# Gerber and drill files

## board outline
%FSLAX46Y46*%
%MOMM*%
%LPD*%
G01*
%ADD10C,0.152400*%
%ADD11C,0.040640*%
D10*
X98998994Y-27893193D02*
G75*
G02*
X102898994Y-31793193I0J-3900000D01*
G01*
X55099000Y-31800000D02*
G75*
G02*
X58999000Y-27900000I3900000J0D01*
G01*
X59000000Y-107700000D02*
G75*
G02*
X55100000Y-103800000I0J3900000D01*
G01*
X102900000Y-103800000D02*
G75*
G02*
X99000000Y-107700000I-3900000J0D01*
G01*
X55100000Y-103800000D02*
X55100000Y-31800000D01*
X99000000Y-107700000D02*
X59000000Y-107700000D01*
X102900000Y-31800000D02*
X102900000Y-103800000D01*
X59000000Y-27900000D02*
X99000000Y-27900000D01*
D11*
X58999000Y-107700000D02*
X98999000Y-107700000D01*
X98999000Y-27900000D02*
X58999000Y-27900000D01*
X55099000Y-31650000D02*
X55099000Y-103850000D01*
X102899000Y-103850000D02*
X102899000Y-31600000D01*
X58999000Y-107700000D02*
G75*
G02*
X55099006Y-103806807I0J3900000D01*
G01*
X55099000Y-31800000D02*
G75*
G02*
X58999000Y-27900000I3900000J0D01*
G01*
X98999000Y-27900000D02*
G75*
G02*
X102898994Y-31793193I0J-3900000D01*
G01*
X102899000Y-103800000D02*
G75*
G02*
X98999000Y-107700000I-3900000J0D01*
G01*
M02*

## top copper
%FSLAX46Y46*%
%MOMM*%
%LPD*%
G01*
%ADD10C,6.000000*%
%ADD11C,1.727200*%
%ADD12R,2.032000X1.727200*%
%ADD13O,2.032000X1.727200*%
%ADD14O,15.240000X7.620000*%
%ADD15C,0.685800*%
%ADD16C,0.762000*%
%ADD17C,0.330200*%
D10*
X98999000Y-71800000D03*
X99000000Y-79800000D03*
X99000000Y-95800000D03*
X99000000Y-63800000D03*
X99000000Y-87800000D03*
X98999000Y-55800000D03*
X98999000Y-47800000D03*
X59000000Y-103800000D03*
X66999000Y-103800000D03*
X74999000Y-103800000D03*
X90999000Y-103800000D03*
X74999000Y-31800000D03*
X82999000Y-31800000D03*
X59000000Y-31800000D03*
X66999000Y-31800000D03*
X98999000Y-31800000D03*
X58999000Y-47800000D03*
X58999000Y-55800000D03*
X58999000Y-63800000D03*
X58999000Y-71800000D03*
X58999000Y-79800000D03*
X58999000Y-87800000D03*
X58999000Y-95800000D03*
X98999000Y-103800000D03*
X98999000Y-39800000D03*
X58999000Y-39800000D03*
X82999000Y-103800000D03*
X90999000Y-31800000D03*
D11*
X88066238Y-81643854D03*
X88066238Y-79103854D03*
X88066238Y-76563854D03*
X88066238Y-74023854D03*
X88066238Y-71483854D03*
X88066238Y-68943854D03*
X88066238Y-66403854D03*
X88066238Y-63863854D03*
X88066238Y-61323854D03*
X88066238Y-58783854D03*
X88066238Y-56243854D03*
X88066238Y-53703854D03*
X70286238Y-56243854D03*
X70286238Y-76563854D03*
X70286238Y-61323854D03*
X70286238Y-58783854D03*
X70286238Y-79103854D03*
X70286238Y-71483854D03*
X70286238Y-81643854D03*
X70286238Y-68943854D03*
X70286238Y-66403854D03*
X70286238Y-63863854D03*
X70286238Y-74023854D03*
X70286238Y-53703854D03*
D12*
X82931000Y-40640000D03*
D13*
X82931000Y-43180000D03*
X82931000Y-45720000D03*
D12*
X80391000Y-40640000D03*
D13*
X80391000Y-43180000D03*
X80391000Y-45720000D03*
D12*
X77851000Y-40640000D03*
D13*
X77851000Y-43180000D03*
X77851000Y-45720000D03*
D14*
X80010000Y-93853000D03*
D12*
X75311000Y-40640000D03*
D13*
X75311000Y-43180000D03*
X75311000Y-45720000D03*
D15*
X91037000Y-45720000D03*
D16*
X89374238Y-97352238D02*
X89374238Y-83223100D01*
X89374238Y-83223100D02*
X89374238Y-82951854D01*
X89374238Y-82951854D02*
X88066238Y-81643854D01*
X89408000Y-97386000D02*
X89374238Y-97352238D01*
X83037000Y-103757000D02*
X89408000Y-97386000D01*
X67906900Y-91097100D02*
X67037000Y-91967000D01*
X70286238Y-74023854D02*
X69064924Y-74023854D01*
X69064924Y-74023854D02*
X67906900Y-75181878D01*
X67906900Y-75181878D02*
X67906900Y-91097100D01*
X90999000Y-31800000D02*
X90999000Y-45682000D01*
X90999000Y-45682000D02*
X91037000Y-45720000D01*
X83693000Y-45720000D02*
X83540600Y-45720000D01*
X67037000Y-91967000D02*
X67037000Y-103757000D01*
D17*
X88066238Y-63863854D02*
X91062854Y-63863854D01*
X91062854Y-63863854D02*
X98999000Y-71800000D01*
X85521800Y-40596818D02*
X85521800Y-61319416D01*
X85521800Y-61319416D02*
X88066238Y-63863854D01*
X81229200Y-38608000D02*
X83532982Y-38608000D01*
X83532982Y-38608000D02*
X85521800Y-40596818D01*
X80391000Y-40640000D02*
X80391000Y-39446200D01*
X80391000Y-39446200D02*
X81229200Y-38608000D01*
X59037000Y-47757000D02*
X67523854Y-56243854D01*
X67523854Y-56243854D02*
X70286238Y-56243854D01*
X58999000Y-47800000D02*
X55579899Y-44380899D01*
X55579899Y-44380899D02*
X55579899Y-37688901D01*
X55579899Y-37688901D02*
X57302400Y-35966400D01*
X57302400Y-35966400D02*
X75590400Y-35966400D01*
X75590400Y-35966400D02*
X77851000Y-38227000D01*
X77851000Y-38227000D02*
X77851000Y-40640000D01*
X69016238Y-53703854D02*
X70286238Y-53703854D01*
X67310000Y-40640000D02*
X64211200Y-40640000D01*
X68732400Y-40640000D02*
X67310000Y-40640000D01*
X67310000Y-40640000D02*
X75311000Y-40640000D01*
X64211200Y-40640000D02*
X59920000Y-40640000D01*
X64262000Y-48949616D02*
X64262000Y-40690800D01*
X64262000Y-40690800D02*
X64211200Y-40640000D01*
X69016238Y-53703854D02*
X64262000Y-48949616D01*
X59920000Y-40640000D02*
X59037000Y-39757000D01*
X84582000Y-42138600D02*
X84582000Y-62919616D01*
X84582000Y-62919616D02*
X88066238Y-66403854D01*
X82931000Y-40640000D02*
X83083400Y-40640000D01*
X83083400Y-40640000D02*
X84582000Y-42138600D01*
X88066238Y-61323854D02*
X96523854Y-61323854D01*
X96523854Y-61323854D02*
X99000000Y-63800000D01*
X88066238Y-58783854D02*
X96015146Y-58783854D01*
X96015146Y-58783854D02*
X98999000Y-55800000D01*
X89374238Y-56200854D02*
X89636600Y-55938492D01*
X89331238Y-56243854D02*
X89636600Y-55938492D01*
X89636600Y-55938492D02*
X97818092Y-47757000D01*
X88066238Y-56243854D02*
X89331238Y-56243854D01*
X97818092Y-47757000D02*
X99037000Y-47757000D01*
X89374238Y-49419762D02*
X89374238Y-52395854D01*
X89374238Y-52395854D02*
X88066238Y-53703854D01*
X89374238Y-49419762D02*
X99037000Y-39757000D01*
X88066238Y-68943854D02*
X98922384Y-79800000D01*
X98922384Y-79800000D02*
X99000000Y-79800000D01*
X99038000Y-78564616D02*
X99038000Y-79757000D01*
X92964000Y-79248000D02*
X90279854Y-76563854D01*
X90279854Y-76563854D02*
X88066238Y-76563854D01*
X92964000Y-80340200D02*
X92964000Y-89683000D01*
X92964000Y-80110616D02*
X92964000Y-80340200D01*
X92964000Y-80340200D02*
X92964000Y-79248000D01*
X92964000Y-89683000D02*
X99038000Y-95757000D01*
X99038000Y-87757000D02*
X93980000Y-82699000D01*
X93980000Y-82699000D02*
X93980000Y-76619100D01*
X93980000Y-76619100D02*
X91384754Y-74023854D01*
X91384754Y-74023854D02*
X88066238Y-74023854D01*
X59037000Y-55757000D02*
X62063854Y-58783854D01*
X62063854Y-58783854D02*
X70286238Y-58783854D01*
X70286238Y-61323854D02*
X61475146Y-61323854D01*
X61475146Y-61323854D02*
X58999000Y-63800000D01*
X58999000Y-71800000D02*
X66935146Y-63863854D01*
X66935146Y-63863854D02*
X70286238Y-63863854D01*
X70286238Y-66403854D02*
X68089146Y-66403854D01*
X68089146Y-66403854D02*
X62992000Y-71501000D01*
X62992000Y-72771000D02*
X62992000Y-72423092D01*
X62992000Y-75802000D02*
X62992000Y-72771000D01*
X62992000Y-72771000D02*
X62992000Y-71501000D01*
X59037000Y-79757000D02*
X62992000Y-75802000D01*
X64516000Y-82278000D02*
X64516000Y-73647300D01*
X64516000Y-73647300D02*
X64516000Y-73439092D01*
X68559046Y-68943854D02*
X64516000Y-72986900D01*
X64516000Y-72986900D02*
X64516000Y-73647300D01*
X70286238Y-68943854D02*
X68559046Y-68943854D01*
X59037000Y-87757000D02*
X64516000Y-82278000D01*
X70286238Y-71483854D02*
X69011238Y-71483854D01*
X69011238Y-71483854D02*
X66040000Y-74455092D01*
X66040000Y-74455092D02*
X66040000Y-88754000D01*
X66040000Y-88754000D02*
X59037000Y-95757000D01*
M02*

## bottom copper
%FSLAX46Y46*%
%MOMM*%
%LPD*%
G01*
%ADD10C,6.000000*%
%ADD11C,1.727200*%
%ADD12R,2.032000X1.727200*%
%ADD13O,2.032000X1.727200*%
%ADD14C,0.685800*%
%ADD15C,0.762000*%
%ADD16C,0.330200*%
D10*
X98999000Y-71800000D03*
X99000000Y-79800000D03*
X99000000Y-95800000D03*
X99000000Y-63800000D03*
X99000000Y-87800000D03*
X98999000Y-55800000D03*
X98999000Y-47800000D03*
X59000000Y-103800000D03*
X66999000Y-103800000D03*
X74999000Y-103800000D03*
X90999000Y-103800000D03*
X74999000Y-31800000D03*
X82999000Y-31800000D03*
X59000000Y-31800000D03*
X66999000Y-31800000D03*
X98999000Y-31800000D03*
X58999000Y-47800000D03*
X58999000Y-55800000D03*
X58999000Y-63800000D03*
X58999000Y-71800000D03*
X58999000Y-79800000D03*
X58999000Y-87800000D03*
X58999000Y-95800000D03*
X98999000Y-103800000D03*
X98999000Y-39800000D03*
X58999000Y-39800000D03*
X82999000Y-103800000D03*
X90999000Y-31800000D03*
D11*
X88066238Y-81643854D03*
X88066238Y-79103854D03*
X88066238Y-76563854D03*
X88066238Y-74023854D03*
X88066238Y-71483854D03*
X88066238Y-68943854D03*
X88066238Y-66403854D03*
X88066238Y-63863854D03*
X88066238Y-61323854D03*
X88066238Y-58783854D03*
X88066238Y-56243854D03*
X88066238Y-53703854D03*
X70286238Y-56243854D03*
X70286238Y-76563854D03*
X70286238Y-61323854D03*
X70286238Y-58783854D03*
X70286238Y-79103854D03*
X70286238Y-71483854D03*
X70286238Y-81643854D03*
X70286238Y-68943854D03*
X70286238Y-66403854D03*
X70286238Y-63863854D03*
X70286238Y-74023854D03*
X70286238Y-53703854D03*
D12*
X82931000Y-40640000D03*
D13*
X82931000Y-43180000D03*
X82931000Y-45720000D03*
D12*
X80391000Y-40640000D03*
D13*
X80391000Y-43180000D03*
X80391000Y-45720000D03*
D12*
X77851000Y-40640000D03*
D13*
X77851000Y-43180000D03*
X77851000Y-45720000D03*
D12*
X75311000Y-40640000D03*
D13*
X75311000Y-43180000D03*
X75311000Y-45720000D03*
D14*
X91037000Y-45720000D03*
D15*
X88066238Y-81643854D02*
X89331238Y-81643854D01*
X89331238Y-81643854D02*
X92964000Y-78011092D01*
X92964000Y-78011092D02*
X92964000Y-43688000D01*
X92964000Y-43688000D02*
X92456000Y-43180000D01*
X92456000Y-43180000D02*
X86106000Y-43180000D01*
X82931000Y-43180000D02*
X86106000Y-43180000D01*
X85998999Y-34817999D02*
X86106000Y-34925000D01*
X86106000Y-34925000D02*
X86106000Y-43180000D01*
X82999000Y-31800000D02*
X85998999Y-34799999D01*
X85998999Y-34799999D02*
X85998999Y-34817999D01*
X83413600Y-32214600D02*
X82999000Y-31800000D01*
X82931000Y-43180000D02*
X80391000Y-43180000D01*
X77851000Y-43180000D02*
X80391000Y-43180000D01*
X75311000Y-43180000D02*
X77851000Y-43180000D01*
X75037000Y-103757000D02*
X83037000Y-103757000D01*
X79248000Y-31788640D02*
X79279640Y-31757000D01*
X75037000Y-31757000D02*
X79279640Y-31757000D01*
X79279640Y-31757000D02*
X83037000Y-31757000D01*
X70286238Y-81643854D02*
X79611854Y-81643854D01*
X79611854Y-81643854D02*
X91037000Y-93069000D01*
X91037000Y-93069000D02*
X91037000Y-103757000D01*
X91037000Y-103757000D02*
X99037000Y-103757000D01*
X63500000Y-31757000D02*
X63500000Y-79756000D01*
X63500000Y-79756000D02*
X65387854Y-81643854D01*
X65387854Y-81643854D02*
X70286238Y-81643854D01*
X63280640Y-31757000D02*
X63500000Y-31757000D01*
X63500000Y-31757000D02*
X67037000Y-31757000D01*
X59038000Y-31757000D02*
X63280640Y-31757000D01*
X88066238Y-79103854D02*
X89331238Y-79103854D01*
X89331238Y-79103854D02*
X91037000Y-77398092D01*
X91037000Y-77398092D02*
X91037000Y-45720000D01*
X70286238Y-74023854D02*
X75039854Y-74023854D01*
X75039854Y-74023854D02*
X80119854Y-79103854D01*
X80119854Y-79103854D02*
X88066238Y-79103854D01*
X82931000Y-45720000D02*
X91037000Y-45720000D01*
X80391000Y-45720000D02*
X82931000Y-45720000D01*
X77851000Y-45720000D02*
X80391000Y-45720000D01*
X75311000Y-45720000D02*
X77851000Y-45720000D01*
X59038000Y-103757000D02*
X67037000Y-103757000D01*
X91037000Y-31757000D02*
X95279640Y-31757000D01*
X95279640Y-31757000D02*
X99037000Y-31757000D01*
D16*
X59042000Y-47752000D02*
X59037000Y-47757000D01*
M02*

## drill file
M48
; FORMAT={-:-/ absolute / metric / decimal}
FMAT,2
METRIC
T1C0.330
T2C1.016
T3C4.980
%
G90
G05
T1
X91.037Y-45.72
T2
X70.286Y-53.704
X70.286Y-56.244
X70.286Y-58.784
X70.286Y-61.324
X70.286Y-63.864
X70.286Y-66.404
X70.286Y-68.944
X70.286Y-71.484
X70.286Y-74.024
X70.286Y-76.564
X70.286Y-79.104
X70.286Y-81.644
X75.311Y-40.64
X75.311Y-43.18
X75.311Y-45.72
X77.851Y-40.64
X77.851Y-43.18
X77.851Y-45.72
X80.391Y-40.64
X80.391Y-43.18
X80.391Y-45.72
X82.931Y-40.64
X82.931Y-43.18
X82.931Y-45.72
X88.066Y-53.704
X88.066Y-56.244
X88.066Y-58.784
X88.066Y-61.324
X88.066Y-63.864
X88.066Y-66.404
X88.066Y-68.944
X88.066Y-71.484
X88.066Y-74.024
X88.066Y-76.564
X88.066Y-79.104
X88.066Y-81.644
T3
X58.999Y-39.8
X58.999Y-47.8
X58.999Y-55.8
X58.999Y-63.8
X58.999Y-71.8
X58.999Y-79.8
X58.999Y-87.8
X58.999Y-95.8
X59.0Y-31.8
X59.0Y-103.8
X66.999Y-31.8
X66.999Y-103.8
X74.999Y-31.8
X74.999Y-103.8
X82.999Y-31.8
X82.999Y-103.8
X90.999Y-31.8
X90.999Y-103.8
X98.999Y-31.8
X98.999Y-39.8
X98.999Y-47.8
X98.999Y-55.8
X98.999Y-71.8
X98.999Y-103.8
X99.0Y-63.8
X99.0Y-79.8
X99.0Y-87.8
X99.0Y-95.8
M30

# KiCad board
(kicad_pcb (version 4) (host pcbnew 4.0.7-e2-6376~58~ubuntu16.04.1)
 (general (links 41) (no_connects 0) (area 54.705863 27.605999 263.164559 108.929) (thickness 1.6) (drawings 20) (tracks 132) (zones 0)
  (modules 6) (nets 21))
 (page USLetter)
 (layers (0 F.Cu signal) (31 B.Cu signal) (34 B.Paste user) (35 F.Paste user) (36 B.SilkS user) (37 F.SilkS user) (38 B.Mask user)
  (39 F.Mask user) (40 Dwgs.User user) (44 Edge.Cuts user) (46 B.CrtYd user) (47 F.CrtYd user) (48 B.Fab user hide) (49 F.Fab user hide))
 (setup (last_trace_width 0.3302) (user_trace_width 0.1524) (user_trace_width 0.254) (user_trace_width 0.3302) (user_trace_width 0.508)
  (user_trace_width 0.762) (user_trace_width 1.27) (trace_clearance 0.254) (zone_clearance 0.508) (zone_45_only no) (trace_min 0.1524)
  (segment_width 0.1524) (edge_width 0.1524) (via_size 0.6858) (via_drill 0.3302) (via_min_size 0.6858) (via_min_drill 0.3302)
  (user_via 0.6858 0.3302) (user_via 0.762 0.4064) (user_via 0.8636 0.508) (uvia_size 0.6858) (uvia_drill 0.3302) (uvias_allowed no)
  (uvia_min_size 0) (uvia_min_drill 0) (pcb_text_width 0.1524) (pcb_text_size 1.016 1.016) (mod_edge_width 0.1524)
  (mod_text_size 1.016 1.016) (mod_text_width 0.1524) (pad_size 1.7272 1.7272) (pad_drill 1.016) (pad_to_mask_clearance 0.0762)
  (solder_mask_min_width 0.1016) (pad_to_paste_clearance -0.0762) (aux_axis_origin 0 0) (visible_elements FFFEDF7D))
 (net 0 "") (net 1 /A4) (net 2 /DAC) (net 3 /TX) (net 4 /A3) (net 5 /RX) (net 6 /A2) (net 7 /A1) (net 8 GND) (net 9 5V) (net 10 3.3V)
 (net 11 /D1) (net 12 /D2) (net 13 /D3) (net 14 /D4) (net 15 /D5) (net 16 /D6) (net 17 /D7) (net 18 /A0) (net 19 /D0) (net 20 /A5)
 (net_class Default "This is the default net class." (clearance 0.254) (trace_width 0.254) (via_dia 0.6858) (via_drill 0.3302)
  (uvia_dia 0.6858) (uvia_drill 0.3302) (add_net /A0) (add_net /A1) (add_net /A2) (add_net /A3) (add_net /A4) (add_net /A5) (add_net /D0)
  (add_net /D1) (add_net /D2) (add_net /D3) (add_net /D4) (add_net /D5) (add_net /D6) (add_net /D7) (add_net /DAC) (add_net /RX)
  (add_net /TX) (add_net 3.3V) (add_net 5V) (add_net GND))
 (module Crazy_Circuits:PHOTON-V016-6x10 (layer F.Cu) (at 58.999 103.8)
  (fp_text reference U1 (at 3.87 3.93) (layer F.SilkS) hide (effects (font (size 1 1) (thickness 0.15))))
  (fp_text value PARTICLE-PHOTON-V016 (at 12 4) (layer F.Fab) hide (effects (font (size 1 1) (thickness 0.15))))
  (fp_line (start 0 3.9) (end 40 3.9) (layer Edge.Cuts) (width 0.04064))
  (fp_line (start 40 -75.9) (end 0 -75.9) (layer Edge.Cuts) (width 0.04064))
  (fp_line (start -3.9 -72.15) (end -3.9 0.05) (layer Edge.Cuts) (width 0.04064))
  (fp_line (start 43.9 0.05) (end 43.9 -72.2) (layer Edge.Cuts) (width 0.04064))
  (fp_arc (start 0 0) (end 0 3.9) (angle 89.9) (layer Edge.Cuts) (width 0.04064))
  (fp_arc (start 0 -72) (end -3.9 -72) (angle 90) (layer Edge.Cuts) (width 0.04064))
  (fp_arc (start 40 -72) (end 40 -75.9) (angle 89.9) (layer Edge.Cuts) (width 0.04064))
  (fp_arc (start 40 0) (end 43.9 0) (angle 90) (layer Edge.Cuts) (width 0.04064))
  (pad A4 thru_hole circle (at 40 -32 90) (size 6 6) (drill 4.98) (layers *.Cu *.Mask) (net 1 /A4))
  (pad DAC thru_hole circle (at 40.001 -24 90) (size 6 6) (drill 4.98) (layers *.Cu *.Mask) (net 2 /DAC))
  (pad TX thru_hole circle (at 40.001 -8 90) (size 6 6) (drill 4.98) (layers *.Cu *.Mask) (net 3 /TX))
  (pad A3 thru_hole circle (at 40.001 -40 90) (size 6 6) (drill 4.98) (layers *.Cu *.Mask) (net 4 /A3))
  (pad RX thru_hole circle (at 40.001 -16 90) (size 6 6) (drill 4.98) (layers *.Cu *.Mask) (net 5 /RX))
  (pad A2 thru_hole circle (at 40 -48 90) (size 6 6) (drill 4.98) (layers *.Cu *.Mask) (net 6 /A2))
  (pad A1 thru_hole circle (at 40 -56 90) (size 6 6) (drill 4.98) (layers *.Cu *.Mask) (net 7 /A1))
  (pad GND thru_hole circle (at 0.001 0 90) (size 6 6) (drill 4.98) (layers *.Cu *.Mask) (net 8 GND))
  (pad GND thru_hole circle (at 8 0 90) (size 6 6) (drill 4.98) (layers *.Cu *.Mask) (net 8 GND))
  (pad 5V thru_hole circle (at 16 0 90) (size 6 6) (drill 4.98) (layers *.Cu *.Mask) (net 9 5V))
  (pad 3V thru_hole circle (at 32 0 90) (size 6 6) (drill 4.98) (layers *.Cu *.Mask) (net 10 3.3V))
  (pad 5V thru_hole circle (at 16 -72 90) (size 6 6) (drill 4.98) (layers *.Cu *.Mask) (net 9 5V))
  (pad 5V thru_hole circle (at 24 -72 90) (size 6 6) (drill 4.98) (layers *.Cu *.Mask) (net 9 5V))
  (pad 3V thru_hole circle (at 0.001 -72 90) (size 6 6) (drill 4.98) (layers *.Cu *.Mask) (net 10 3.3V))
  (pad 3V thru_hole circle (at 8 -72 90) (size 6 6) (drill 4.98) (layers *.Cu *.Mask) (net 10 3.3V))
  (pad GND thru_hole circle (at 40 -72 90) (size 6 6) (drill 4.98) (layers *.Cu *.Mask) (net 8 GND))
  (pad D1 thru_hole circle (at 0 -56 90) (size 6 6) (drill 4.98) (layers *.Cu *.Mask) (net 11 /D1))
  (pad D2 thru_hole circle (at 0 -48 90) (size 6 6) (drill 4.98) (layers *.Cu *.Mask) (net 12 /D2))
  (pad D3 thru_hole circle (at 0 -40 90) (size 6 6) (drill 4.98) (layers *.Cu *.Mask) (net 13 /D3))
  (pad D4 thru_hole circle (at 0 -32 90) (size 6 6) (drill 4.98) (layers *.Cu *.Mask) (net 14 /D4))
  (pad D5 thru_hole circle (at 0 -24 90) (size 6 6) (drill 4.98) (layers *.Cu *.Mask) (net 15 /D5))
  (pad D6 thru_hole circle (at 0 -16 90) (size 6 6) (drill 4.98) (layers *.Cu *.Mask) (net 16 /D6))
  (pad D7 thru_hole circle (at 0 -8 90) (size 6 6) (drill 4.98) (layers *.Cu *.Mask) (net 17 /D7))
  (pad 3V thru_hole circle (at 40 0 90) (size 6 6) (drill 4.98) (layers *.Cu *.Mask) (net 10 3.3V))
  (pad A0 thru_hole circle (at 40 -64 90) (size 6 6) (drill 4.98) (layers *.Cu *.Mask) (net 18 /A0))
  (pad D0 thru_hole circle (at 0 -64 90) (size 6 6) (drill 4.98) (layers *.Cu *.Mask) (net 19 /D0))
  (pad 5V thru_hole circle (at 24 0 90) (size 6 6) (drill 4.98) (layers *.Cu *.Mask) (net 9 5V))
  (pad GND thru_hole circle (at 32 -72 90) (size 6 6) (drill 4.98) (layers *.Cu *.Mask) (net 8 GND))
  (pad VIN thru_hole circle (at 29.067238 -22.156146 180) (size 1.7272 1.7272) (drill 1.016) (layers *.Cu *.Mask F.SilkS) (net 9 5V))
  (pad GND thru_hole circle (at 29.067238 -24.696146 180) (size 1.7272 1.7272) (drill 1.016) (layers *.Cu *.Mask F.SilkS) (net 8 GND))
  (pad TX thru_hole circle (at 29.067238 -27.236146 180) (size 1.7272 1.7272) (drill 1.016) (layers *.Cu *.Mask F.SilkS) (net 3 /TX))
  (pad RX thru_hole circle (at 29.067238 -29.776146 180) (size 1.7272 1.7272) (drill 1.016) (layers *.Cu *.Mask F.SilkS) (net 5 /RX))
  (pad WKP thru_hole circle (at 29.067238 -32.316146 180) (size 1.7272 1.7272) (drill 1.016) (layers *.Cu *.Mask F.SilkS))
  (pad DAC thru_hole circle (at 29.067238 -34.856146 180) (size 1.7272 1.7272) (drill 1.016) (layers *.Cu *.Mask F.SilkS) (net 2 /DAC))
  (pad A5 thru_hole circle (at 29.067238 -37.396146 180) (size 1.7272 1.7272) (drill 1.016) (layers *.Cu *.Mask F.SilkS) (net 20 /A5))
  (pad A4 thru_hole circle (at 29.067238 -39.936146 180) (size 1.7272 1.7272) (drill 1.016) (layers *.Cu *.Mask F.SilkS) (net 1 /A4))
  (pad A3 thru_hole circle (at 29.067238 -42.476146 180) (size 1.7272 1.7272) (drill 1.016) (layers *.Cu *.Mask F.SilkS) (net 4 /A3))
  (pad A2 thru_hole circle (at 29.067238 -45.016146 180) (size 1.7272 1.7272) (drill 1.016) (layers *.Cu *.Mask F.SilkS) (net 6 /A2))
  (pad A1 thru_hole circle (at 29.067238 -47.556146 180) (size 1.7272 1.7272) (drill 1.016) (layers *.Cu *.Mask F.SilkS) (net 7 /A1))
  (pad A0 thru_hole circle (at 29.067238 -50.096146 180) (size 1.7272 1.7272) (drill 1.016) (layers *.Cu *.Mask F.SilkS) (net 18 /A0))
  (pad D1 thru_hole circle (at 11.287238 -47.556146 180) (size 1.7272 1.7272) (drill 1.016) (layers *.Cu *.Mask F.SilkS) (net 11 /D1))
  (pad VBAT thru_hole circle (at 11.287238 -27.236146 180) (size 1.7272 1.7272) (drill 1.016) (layers *.Cu *.Mask F.SilkS))
  (pad D3 thru_hole circle (at 11.287238 -42.476146 180) (size 1.7272 1.7272) (drill 1.016) (layers *.Cu *.Mask F.SilkS) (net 13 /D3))
  (pad D2 thru_hole circle (at 11.287238 -45.016146 180) (size 1.7272 1.7272) (drill 1.016) (layers *.Cu *.Mask F.SilkS) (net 12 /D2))
  (pad RST thru_hole circle (at 11.287238 -24.696146 180) (size 1.7272 1.7272) (drill 1.016) (layers *.Cu *.Mask F.SilkS))
  (pad D7 thru_hole circle (at 11.287238 -32.316146 180) (size 1.7272 1.7272) (drill 1.016) (layers *.Cu *.Mask F.SilkS) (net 17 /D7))
  (pad 3V thru_hole circle (at 11.287238 -22.156146 180) (size 1.7272 1.7272) (drill 1.016) (layers *.Cu *.Mask F.SilkS) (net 10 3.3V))
  (pad D6 thru_hole circle (at 11.287238 -34.856146 180) (size 1.7272 1.7272) (drill 1.016) (layers *.Cu *.Mask F.SilkS) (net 16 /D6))
  (pad D5 thru_hole circle (at 11.287238 -37.396146 180) (size 1.7272 1.7272) (drill 1.016) (layers *.Cu *.Mask F.SilkS) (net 15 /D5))
  (pad D4 thru_hole circle (at 11.287238 -39.936146 180) (size 1.7272 1.7272) (drill 1.016) (layers *.Cu *.Mask F.SilkS) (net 14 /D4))
  (pad GND thru_hole circle (at 11.287238 -29.776146 180) (size 1.7272 1.7272) (drill 1.016) (layers *.Cu *.Mask F.SilkS) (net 8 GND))
  (pad D0 thru_hole circle (at 11.287238 -50.096146 180) (size 1.7272 1.7272) (drill 1.016) (layers *.Cu *.Mask F.SilkS) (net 19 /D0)))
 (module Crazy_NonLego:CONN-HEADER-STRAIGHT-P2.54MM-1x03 (layer F.Cu) (at 82.931 40.64)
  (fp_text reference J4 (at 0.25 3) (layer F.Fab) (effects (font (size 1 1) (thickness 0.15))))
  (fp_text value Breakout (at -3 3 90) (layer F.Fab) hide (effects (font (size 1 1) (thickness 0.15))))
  (pad A5 thru_hole rect (at 0 0) (size 2.032 1.7272) (drill 1.016) (layers *.Cu *.Mask F.SilkS) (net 20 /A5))
  (pad VIN thru_hole oval (at 0 2.54) (size 2.032 1.7272) (drill 1.016) (layers *.Cu *.Mask F.SilkS) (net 9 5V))
  (pad GND thru_hole oval (at 0 5.08) (size 2.032 1.7272) (drill 1.016) (layers *.Cu *.Mask F.SilkS) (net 8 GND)))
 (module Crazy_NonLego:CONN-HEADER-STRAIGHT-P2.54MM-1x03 (layer F.Cu) (at 80.391 40.64)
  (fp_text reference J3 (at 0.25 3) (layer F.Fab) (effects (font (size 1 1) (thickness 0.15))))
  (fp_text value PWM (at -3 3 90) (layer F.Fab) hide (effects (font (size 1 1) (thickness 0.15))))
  (pad A4 thru_hole rect (at 0 0) (size 2.032 1.7272) (drill 1.016) (layers *.Cu *.Mask F.SilkS) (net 1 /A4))
  (pad VIN thru_hole oval (at 0 2.54) (size 2.032 1.7272) (drill 1.016) (layers *.Cu *.Mask F.SilkS) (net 9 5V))
  (pad GND thru_hole oval (at 0 5.08) (size 2.032 1.7272) (drill 1.016) (layers *.Cu *.Mask F.SilkS) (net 8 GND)))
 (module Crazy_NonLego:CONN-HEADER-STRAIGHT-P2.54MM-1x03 (layer F.Cu) (at 77.851 40.64)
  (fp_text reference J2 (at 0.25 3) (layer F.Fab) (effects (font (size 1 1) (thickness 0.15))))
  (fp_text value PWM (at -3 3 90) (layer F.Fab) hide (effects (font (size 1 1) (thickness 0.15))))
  (pad D1 thru_hole rect (at 0 0) (size 2.032 1.7272) (drill 1.016) (layers *.Cu *.Mask F.SilkS) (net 11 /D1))
  (pad VIN thru_hole oval (at 0 2.54) (size 2.032 1.7272) (drill 1.016) (layers *.Cu *.Mask F.SilkS) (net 9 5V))
  (pad GND thru_hole oval (at 0 5.08) (size 2.032 1.7272) (drill 1.016) (layers *.Cu *.Mask F.SilkS) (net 8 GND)))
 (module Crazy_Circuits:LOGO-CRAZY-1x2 (layer F.Cu) (at 80.01 97.79)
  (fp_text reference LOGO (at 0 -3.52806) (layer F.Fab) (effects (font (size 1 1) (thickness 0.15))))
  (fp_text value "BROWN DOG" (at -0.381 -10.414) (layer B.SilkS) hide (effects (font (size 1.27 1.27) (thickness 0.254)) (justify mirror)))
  (pad BG smd oval (at 0 -3.937) (size 15.24 7.62) (layers F.Cu)))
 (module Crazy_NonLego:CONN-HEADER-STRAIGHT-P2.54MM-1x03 (layer F.Cu) (at 75.311 40.64)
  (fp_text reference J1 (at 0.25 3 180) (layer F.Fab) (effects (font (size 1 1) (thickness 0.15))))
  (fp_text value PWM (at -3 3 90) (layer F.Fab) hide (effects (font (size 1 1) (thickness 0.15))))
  (pad D0 thru_hole rect (at 0 0) (size 2.032 1.7272) (drill 1.016) (layers *.Cu *.Mask F.SilkS) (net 19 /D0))
  (pad VIN thru_hole oval (at 0 2.54) (size 2.032 1.7272) (drill 1.016) (layers *.Cu *.Mask F.SilkS) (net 9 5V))
  (pad GND thru_hole oval (at 0 5.08) (size 2.032 1.7272) (drill 1.016) (layers *.Cu *.Mask F.SilkS) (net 8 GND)))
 (gr_arc (start 98.998994 31.793193) (end 98.998994 27.893193) (angle 90) (layer Edge.Cuts) (width 0.1524))
 (gr_arc (start 58.999 31.8) (end 55.099 31.8) (angle 90) (layer Edge.Cuts) (width 0.1524))
 (gr_arc (start 59 103.8) (end 59 107.7) (angle 90) (layer Edge.Cuts) (width 0.1524))
 (gr_arc (start 99 103.8) (end 102.9 103.8) (angle 90) (layer Edge.Cuts) (width 0.1524))
 (gr_line (start 55.1 103.8) (end 55.1 31.8) (layer Edge.Cuts) (width 0.1524))
 (gr_line (start 99 107.7) (end 59 107.7) (layer Edge.Cuts) (width 0.1524))
 (gr_line (start 102.9 31.8) (end 102.9 103.8) (layer Edge.Cuts) (width 0.1524))
 (gr_line (start 59 27.9) (end 99 27.9) (layer Edge.Cuts) (width 0.1524))
 (segment (start 89.374238 97.352238) (end 89.374238 83.2231) (width 0.762) (layer F.Cu) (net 9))
 (segment (start 89.374238 83.2231) (end 89.374238 82.951854) (width 0.762) (layer F.Cu) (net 9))
 (segment (start 89.374238 82.951854) (end 88.066238 81.643854) (width 0.762) (layer F.Cu) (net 9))
 (segment (start 88.066238 81.643854) (end 89.331238 81.643854) (width 0.762) (layer B.Cu) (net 9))
 (segment (start 89.331238 81.643854) (end 92.964 78.011092) (width 0.762) (layer B.Cu) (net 9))
 (segment (start 92.964 78.011092) (end 92.964 43.688) (width 0.762) (layer B.Cu) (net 9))
 (segment (start 92.964 43.688) (end 92.456 43.18) (width 0.762) (layer B.Cu) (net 9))
 (segment (start 92.456 43.18) (end 86.106 43.18) (width 0.762) (layer B.Cu) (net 9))
 (segment (start 82.931 43.18) (end 86.106 43.18) (width 0.762) (layer B.Cu) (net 9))
 (segment (start 85.998999 34.817999) (end 86.106 34.925) (width 0.762) (layer B.Cu) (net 9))
 (segment (start 86.106 34.925) (end 86.106 43.18) (width 0.762) (layer B.Cu) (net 9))
 (segment (start 82.999 31.8) (end 85.998999 34.799999) (width 0.762) (layer B.Cu) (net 9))
 (segment (start 85.998999 34.799999) (end 85.998999 34.817999) (width 0.762) (layer B.Cu) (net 9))
 (segment (start 83.4136 32.2146) (end 82.999 31.8) (width 0.762) (layer B.Cu) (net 9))
 (segment (start 82.931 43.18) (end 80.391 43.18) (width 0.762) (layer B.Cu) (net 9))
 (segment (start 77.851 43.18) (end 80.391 43.18) (width 0.762) (layer B.Cu) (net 9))
 (segment (start 75.311 43.18) (end 77.851 43.18) (width 0.762) (layer B.Cu) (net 9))
 (segment (start 89.408 97.386) (end 89.374238 97.352238) (width 0.762) (layer F.Cu) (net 9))
 (segment (start 83.037 103.757) (end 89.408 97.386) (width 0.762) (layer F.Cu) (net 9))
 (segment (start 75.037 103.757) (end 83.037 103.757) (width 0.762) (layer B.Cu) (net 9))
 (segment (start 79.248 31.78864) (end 79.27964 31.757) (width 0.762) (layer B.Cu) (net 9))
 (segment (start 75.037 31.757) (end 79.27964 31.757) (width 0.762) (layer B.Cu) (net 9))
 (segment (start 79.27964 31.757) (end 83.037 31.757) (width 0.762) (layer B.Cu) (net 9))
 (segment (start 70.286238 81.643854) (end 79.611854 81.643854) (width 0.762) (layer B.Cu) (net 10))
 (segment (start 79.611854 81.643854) (end 91.037 93.069) (width 0.762) (layer B.Cu) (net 10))
 (segment (start 91.037 93.069) (end 91.037 103.757) (width 0.762) (layer B.Cu) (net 10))
 (segment (start 91.037 103.757) (end 99.037 103.757) (width 0.762) (layer B.Cu) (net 10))
 (segment (start 63.5 31.757) (end 63.5 79.756) (width 0.762) (layer B.Cu) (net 10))
 (segment (start 63.5 79.756) (end 65.387854 81.643854) (width 0.762) (layer B.Cu) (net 10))
 (segment (start 65.387854 81.643854) (end 70.286238 81.643854) (width 0.762) (layer B.Cu) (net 10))
 (segment (start 63.28064 31.757) (end 63.5 31.757) (width 0.762) (layer B.Cu) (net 10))
 (segment (start 63.5 31.757) (end 67.037 31.757) (width 0.762) (layer B.Cu) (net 10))
 (segment (start 59.038 31.757) (end 63.28064 31.757) (width 0.762) (layer B.Cu) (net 10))
 (segment (start 88.066238 79.103854) (end 89.331238 79.103854) (width 0.762) (layer B.Cu) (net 8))
 (segment (start 89.331238 79.103854) (end 91.037 77.398092) (width 0.762) (layer B.Cu) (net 8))
 (segment (start 91.037 77.398092) (end 91.037 45.72) (width 0.762) (layer B.Cu) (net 8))
 (segment (start 70.286238 74.023854) (end 75.039854 74.023854) (width 0.762) (layer B.Cu) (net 8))
 (segment (start 75.039854 74.023854) (end 80.119854 79.103854) (width 0.762) (layer B.Cu) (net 8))
 (segment (start 80.119854 79.103854) (end 88.066238 79.103854) (width 0.762) (layer B.Cu) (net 8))
 (segment (start 67.9069 91.0971) (end 67.037 91.967) (width 0.762) (layer F.Cu) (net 8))
 (segment (start 70.286238 74.023854) (end 69.064924 74.023854) (width 0.762) (layer F.Cu) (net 8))
 (segment (start 69.064924 74.023854) (end 67.9069 75.181878) (width 0.762) (layer F.Cu) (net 8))
 (segment (start 67.9069 75.181878) (end 67.9069 91.0971) (width 0.762) (layer F.Cu) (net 8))
 (segment (start 82.931 45.72) (end 91.037 45.72) (width 0.762) (layer B.Cu) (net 8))
 (segment (start 90.999 31.8) (end 90.999 45.682) (width 0.762) (layer F.Cu) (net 8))
 (segment (start 90.999 45.682) (end 91.037 45.72) (width 0.762) (layer F.Cu) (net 8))
 (via (at 91.037 45.72) (size 0.6858) (drill 0.3302) (layers F.Cu B.Cu) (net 8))
 (segment (start 80.391 45.72) (end 82.931 45.72) (width 0.762) (layer B.Cu) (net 8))
 (segment (start 77.851 45.72) (end 80.391 45.72) (width 0.762) (layer B.Cu) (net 8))
 (segment (start 75.311 45.72) (end 77.851 45.72) (width 0.762) (layer B.Cu) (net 8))
 (segment (start 83.693 45.72) (end 83.5406 45.72) (width 0.762) (layer F.Cu) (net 8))
 (segment (start 67.037 91.967) (end 67.037 103.757) (width 0.762) (layer F.Cu) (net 8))
 (segment (start 59.038 103.757) (end 67.037 103.757) (width 0.762) (layer B.Cu) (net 8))
 (segment (start 91.037 31.757) (end 95.27964 31.757) (width 0.762) (layer B.Cu) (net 8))
 (segment (start 95.27964 31.757) (end 99.037 31.757) (width 0.762) (layer B.Cu) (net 8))
 (segment (start 88.066238 63.863854) (end 91.062854 63.863854) (width 0.3302) (layer F.Cu) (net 1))
 (segment (start 91.062854 63.863854) (end 98.999 71.8) (width 0.3302) (layer F.Cu) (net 1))
 (segment (start 85.5218 40.596818) (end 85.5218 61.319416) (width 0.3302) (layer F.Cu) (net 1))
 (segment (start 85.5218 61.319416) (end 88.066238 63.863854) (width 0.3302) (layer F.Cu) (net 1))
 (segment (start 81.2292 38.608) (end 83.532982 38.608) (width 0.3302) (layer F.Cu) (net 1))
 (segment (start 83.532982 38.608) (end 85.5218 40.596818) (width 0.3302) (layer F.Cu) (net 1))
 (segment (start 80.391 40.64) (end 80.391 39.4462) (width 0.3302) (layer F.Cu) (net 1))
 (segment (start 80.391 39.4462) (end 81.2292 38.608) (width 0.3302) (layer F.Cu) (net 1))
 (segment (start 59.037 47.757) (end 67.523854 56.243854) (width 0.3302) (layer F.Cu) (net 11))
 (segment (start 67.523854 56.243854) (end 70.286238 56.243854) (width 0.3302) (layer F.Cu) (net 11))
 (segment (start 58.999 47.8) (end 55.579899 44.380899) (width 0.3302) (layer F.Cu) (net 11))
 (segment (start 55.579899 44.380899) (end 55.579899 37.688901) (width 0.3302) (layer F.Cu) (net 11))
 (segment (start 55.579899 37.688901) (end 57.3024 35.9664) (width 0.3302) (layer F.Cu) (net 11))
 (segment (start 57.3024 35.9664) (end 75.5904 35.9664) (width 0.3302) (layer F.Cu) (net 11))
 (segment (start 75.5904 35.9664) (end 77.851 38.227) (width 0.3302) (layer F.Cu) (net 11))
 (segment (start 77.851 38.227) (end 77.851 40.64) (width 0.3302) (layer F.Cu) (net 11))
 (segment (start 59.042 47.752) (end 59.037 47.757) (width 0.3302) (layer B.Cu) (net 11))
 (segment (start 69.016238 53.703854) (end 70.286238 53.703854) (width 0.3302) (layer F.Cu) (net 19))
 (segment (start 67.31 40.64) (end 64.2112 40.64) (width 0.3302) (layer F.Cu) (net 19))
 (segment (start 68.7324 40.64) (end 67.31 40.64) (width 0.3302) (layer F.Cu) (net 19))
 (segment (start 67.31 40.64) (end 75.311 40.64) (width 0.3302) (layer F.Cu) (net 19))
 (segment (start 64.2112 40.64) (end 59.92 40.64) (width 0.3302) (layer F.Cu) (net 19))
 (segment (start 64.262 48.949616) (end 64.262 40.6908) (width 0.3302) (layer F.Cu) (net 19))
 (segment (start 64.262 40.6908) (end 64.2112 40.64) (width 0.3302) (layer F.Cu) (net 19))
 (segment (start 69.016238 53.703854) (end 64.262 48.949616) (width 0.3302) (layer F.Cu) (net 19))
 (segment (start 59.92 40.64) (end 59.037 39.757) (width 0.3302) (layer F.Cu) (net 19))
 (segment (start 84.582 42.1386) (end 84.582 62.919616) (width 0.3302) (layer F.Cu) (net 20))
 (segment (start 84.582 62.919616) (end 88.066238 66.403854) (width 0.3302) (layer F.Cu) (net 20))
 (segment (start 82.931 40.64) (end 83.0834 40.64) (width 0.3302) (layer F.Cu) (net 20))
 (segment (start 83.0834 40.64) (end 84.582 42.1386) (width 0.3302) (layer F.Cu) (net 20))
 (segment (start 88.066238 61.323854) (end 96.523854 61.323854) (width 0.3302) (layer F.Cu) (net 4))
 (segment (start 96.523854 61.323854) (end 99 63.8) (width 0.3302) (layer F.Cu) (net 4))
 (segment (start 88.066238 58.783854) (end 96.015146 58.783854) (width 0.3302) (layer F.Cu) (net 6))
 (segment (start 96.015146 58.783854) (end 98.999 55.8) (width 0.3302) (layer F.Cu) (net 6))
 (segment (start 89.374238 56.200854) (end 89.6366 55.938492) (width 0.3302) (layer F.Cu) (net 7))
 (segment (start 89.331238 56.243854) (end 89.6366 55.938492) (width 0.3302) (layer F.Cu) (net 7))
 (segment (start 89.6366 55.938492) (end 97.818092 47.757) (width 0.3302) (layer F.Cu) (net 7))
 (segment (start 88.066238 56.243854) (end 89.331238 56.243854) (width 0.3302) (layer F.Cu) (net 7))
 (segment (start 97.818092 47.757) (end 99.037 47.757) (width 0.3302) (layer F.Cu) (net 7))
 (segment (start 89.374238 49.419762) (end 89.374238 52.395854) (width 0.3302) (layer F.Cu) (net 18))
 (segment (start 89.374238 52.395854) (end 88.066238 53.703854) (width 0.3302) (layer F.Cu) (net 18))
 (segment (start 89.374238 49.419762) (end 99.037 39.757) (width 0.3302) (layer F.Cu) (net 18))
 (segment (start 88.066238 68.943854) (end 98.922384 79.8) (width 0.3302) (layer F.Cu) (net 2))
 (segment (start 98.922384 79.8) (end 99 79.8) (width 0.3302) (layer F.Cu) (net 2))
 (segment (start 99.038 78.564616) (end 99.038 79.757) (width 0.3302) (layer F.Cu) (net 2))
 (segment (start 92.964 79.248) (end 90.279854 76.563854) (width 0.3302) (layer F.Cu) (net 3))
 (segment (start 90.279854 76.563854) (end 88.066238 76.563854) (width 0.3302) (layer F.Cu) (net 3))
 (segment (start 92.964 80.3402) (end 92.964 89.683) (width 0.3302) (layer F.Cu) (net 3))
 (segment (start 92.964 80.110616) (end 92.964 80.3402) (width 0.3302) (layer F.Cu) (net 3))
 (segment (start 92.964 80.3402) (end 92.964 79.248) (width 0.3302) (layer F.Cu) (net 3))
 (segment (start 92.964 89.683) (end 99.038 95.757) (width 0.3302) (layer F.Cu) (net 3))
 (segment (start 99.038 87.757) (end 93.98 82.699) (width 0.3302) (layer F.Cu) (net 5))
 (segment (start 93.98 82.699) (end 93.98 76.6191) (width 0.3302) (layer F.Cu) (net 5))
 (segment (start 93.98 76.6191) (end 91.384754 74.023854) (width 0.3302) (layer F.Cu) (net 5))
 (segment (start 91.384754 74.023854) (end 88.066238 74.023854) (width 0.3302) (layer F.Cu) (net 5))
 (segment (start 59.037 55.757) (end 62.063854 58.783854) (width 0.3302) (layer F.Cu) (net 12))
 (segment (start 62.063854 58.783854) (end 70.286238 58.783854) (width 0.3302) (layer F.Cu) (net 12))
 (segment (start 70.286238 61.323854) (end 61.475146 61.323854) (width 0.3302) (layer F.Cu) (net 13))
 (segment (start 61.475146 61.323854) (end 58.999 63.8) (width 0.3302) (layer F.Cu) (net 13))
 (segment (start 58.999 71.8) (end 66.935146 63.863854) (width 0.3302) (layer F.Cu) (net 14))
 (segment (start 66.935146 63.863854) (end 70.286238 63.863854) (width 0.3302) (layer F.Cu) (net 14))
 (segment (start 70.286238 66.403854) (end 68.089146 66.403854) (width 0.3302) (layer F.Cu) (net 15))
 (segment (start 68.089146 66.403854) (end 62.992 71.501) (width 0.3302) (layer F.Cu) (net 15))
 (segment (start 62.992 72.771) (end 62.992 72.423092) (width 0.3302) (layer F.Cu) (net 15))
 (segment (start 62.992 75.802) (end 62.992 72.771) (width 0.3302) (layer F.Cu) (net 15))
 (segment (start 62.992 72.771) (end 62.992 71.501) (width 0.3302) (layer F.Cu) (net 15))
 (segment (start 59.037 79.757) (end 62.992 75.802) (width 0.3302) (layer F.Cu) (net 15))
 (segment (start 64.516 82.278) (end 64.516 73.6473) (width 0.3302) (layer F.Cu) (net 16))
 (segment (start 64.516 73.6473) (end 64.516 73.439092) (width 0.3302) (layer F.Cu) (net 16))
 (segment (start 68.559046 68.943854) (end 64.516 72.9869) (width 0.3302) (layer F.Cu) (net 16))
 (segment (start 64.516 72.9869) (end 64.516 73.6473) (width 0.3302) (layer F.Cu) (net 16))
 (segment (start 70.286238 68.943854) (end 68.559046 68.943854) (width 0.3302) (layer F.Cu) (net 16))
 (segment (start 59.037 87.757) (end 64.516 82.278) (width 0.3302) (layer F.Cu) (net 16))
 (segment (start 70.286238 71.483854) (end 69.011238 71.483854) (width 0.3302) (layer F.Cu) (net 17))
 (segment (start 69.011238 71.483854) (end 66.04 74.455092) (width 0.3302) (layer F.Cu) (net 17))
 (segment (start 66.04 74.455092) (end 66.04 88.754) (width 0.3302) (layer F.Cu) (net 17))
 (segment (start 66.04 88.754) (end 59.037 95.757) (width 0.3302) (layer F.Cu) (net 17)))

